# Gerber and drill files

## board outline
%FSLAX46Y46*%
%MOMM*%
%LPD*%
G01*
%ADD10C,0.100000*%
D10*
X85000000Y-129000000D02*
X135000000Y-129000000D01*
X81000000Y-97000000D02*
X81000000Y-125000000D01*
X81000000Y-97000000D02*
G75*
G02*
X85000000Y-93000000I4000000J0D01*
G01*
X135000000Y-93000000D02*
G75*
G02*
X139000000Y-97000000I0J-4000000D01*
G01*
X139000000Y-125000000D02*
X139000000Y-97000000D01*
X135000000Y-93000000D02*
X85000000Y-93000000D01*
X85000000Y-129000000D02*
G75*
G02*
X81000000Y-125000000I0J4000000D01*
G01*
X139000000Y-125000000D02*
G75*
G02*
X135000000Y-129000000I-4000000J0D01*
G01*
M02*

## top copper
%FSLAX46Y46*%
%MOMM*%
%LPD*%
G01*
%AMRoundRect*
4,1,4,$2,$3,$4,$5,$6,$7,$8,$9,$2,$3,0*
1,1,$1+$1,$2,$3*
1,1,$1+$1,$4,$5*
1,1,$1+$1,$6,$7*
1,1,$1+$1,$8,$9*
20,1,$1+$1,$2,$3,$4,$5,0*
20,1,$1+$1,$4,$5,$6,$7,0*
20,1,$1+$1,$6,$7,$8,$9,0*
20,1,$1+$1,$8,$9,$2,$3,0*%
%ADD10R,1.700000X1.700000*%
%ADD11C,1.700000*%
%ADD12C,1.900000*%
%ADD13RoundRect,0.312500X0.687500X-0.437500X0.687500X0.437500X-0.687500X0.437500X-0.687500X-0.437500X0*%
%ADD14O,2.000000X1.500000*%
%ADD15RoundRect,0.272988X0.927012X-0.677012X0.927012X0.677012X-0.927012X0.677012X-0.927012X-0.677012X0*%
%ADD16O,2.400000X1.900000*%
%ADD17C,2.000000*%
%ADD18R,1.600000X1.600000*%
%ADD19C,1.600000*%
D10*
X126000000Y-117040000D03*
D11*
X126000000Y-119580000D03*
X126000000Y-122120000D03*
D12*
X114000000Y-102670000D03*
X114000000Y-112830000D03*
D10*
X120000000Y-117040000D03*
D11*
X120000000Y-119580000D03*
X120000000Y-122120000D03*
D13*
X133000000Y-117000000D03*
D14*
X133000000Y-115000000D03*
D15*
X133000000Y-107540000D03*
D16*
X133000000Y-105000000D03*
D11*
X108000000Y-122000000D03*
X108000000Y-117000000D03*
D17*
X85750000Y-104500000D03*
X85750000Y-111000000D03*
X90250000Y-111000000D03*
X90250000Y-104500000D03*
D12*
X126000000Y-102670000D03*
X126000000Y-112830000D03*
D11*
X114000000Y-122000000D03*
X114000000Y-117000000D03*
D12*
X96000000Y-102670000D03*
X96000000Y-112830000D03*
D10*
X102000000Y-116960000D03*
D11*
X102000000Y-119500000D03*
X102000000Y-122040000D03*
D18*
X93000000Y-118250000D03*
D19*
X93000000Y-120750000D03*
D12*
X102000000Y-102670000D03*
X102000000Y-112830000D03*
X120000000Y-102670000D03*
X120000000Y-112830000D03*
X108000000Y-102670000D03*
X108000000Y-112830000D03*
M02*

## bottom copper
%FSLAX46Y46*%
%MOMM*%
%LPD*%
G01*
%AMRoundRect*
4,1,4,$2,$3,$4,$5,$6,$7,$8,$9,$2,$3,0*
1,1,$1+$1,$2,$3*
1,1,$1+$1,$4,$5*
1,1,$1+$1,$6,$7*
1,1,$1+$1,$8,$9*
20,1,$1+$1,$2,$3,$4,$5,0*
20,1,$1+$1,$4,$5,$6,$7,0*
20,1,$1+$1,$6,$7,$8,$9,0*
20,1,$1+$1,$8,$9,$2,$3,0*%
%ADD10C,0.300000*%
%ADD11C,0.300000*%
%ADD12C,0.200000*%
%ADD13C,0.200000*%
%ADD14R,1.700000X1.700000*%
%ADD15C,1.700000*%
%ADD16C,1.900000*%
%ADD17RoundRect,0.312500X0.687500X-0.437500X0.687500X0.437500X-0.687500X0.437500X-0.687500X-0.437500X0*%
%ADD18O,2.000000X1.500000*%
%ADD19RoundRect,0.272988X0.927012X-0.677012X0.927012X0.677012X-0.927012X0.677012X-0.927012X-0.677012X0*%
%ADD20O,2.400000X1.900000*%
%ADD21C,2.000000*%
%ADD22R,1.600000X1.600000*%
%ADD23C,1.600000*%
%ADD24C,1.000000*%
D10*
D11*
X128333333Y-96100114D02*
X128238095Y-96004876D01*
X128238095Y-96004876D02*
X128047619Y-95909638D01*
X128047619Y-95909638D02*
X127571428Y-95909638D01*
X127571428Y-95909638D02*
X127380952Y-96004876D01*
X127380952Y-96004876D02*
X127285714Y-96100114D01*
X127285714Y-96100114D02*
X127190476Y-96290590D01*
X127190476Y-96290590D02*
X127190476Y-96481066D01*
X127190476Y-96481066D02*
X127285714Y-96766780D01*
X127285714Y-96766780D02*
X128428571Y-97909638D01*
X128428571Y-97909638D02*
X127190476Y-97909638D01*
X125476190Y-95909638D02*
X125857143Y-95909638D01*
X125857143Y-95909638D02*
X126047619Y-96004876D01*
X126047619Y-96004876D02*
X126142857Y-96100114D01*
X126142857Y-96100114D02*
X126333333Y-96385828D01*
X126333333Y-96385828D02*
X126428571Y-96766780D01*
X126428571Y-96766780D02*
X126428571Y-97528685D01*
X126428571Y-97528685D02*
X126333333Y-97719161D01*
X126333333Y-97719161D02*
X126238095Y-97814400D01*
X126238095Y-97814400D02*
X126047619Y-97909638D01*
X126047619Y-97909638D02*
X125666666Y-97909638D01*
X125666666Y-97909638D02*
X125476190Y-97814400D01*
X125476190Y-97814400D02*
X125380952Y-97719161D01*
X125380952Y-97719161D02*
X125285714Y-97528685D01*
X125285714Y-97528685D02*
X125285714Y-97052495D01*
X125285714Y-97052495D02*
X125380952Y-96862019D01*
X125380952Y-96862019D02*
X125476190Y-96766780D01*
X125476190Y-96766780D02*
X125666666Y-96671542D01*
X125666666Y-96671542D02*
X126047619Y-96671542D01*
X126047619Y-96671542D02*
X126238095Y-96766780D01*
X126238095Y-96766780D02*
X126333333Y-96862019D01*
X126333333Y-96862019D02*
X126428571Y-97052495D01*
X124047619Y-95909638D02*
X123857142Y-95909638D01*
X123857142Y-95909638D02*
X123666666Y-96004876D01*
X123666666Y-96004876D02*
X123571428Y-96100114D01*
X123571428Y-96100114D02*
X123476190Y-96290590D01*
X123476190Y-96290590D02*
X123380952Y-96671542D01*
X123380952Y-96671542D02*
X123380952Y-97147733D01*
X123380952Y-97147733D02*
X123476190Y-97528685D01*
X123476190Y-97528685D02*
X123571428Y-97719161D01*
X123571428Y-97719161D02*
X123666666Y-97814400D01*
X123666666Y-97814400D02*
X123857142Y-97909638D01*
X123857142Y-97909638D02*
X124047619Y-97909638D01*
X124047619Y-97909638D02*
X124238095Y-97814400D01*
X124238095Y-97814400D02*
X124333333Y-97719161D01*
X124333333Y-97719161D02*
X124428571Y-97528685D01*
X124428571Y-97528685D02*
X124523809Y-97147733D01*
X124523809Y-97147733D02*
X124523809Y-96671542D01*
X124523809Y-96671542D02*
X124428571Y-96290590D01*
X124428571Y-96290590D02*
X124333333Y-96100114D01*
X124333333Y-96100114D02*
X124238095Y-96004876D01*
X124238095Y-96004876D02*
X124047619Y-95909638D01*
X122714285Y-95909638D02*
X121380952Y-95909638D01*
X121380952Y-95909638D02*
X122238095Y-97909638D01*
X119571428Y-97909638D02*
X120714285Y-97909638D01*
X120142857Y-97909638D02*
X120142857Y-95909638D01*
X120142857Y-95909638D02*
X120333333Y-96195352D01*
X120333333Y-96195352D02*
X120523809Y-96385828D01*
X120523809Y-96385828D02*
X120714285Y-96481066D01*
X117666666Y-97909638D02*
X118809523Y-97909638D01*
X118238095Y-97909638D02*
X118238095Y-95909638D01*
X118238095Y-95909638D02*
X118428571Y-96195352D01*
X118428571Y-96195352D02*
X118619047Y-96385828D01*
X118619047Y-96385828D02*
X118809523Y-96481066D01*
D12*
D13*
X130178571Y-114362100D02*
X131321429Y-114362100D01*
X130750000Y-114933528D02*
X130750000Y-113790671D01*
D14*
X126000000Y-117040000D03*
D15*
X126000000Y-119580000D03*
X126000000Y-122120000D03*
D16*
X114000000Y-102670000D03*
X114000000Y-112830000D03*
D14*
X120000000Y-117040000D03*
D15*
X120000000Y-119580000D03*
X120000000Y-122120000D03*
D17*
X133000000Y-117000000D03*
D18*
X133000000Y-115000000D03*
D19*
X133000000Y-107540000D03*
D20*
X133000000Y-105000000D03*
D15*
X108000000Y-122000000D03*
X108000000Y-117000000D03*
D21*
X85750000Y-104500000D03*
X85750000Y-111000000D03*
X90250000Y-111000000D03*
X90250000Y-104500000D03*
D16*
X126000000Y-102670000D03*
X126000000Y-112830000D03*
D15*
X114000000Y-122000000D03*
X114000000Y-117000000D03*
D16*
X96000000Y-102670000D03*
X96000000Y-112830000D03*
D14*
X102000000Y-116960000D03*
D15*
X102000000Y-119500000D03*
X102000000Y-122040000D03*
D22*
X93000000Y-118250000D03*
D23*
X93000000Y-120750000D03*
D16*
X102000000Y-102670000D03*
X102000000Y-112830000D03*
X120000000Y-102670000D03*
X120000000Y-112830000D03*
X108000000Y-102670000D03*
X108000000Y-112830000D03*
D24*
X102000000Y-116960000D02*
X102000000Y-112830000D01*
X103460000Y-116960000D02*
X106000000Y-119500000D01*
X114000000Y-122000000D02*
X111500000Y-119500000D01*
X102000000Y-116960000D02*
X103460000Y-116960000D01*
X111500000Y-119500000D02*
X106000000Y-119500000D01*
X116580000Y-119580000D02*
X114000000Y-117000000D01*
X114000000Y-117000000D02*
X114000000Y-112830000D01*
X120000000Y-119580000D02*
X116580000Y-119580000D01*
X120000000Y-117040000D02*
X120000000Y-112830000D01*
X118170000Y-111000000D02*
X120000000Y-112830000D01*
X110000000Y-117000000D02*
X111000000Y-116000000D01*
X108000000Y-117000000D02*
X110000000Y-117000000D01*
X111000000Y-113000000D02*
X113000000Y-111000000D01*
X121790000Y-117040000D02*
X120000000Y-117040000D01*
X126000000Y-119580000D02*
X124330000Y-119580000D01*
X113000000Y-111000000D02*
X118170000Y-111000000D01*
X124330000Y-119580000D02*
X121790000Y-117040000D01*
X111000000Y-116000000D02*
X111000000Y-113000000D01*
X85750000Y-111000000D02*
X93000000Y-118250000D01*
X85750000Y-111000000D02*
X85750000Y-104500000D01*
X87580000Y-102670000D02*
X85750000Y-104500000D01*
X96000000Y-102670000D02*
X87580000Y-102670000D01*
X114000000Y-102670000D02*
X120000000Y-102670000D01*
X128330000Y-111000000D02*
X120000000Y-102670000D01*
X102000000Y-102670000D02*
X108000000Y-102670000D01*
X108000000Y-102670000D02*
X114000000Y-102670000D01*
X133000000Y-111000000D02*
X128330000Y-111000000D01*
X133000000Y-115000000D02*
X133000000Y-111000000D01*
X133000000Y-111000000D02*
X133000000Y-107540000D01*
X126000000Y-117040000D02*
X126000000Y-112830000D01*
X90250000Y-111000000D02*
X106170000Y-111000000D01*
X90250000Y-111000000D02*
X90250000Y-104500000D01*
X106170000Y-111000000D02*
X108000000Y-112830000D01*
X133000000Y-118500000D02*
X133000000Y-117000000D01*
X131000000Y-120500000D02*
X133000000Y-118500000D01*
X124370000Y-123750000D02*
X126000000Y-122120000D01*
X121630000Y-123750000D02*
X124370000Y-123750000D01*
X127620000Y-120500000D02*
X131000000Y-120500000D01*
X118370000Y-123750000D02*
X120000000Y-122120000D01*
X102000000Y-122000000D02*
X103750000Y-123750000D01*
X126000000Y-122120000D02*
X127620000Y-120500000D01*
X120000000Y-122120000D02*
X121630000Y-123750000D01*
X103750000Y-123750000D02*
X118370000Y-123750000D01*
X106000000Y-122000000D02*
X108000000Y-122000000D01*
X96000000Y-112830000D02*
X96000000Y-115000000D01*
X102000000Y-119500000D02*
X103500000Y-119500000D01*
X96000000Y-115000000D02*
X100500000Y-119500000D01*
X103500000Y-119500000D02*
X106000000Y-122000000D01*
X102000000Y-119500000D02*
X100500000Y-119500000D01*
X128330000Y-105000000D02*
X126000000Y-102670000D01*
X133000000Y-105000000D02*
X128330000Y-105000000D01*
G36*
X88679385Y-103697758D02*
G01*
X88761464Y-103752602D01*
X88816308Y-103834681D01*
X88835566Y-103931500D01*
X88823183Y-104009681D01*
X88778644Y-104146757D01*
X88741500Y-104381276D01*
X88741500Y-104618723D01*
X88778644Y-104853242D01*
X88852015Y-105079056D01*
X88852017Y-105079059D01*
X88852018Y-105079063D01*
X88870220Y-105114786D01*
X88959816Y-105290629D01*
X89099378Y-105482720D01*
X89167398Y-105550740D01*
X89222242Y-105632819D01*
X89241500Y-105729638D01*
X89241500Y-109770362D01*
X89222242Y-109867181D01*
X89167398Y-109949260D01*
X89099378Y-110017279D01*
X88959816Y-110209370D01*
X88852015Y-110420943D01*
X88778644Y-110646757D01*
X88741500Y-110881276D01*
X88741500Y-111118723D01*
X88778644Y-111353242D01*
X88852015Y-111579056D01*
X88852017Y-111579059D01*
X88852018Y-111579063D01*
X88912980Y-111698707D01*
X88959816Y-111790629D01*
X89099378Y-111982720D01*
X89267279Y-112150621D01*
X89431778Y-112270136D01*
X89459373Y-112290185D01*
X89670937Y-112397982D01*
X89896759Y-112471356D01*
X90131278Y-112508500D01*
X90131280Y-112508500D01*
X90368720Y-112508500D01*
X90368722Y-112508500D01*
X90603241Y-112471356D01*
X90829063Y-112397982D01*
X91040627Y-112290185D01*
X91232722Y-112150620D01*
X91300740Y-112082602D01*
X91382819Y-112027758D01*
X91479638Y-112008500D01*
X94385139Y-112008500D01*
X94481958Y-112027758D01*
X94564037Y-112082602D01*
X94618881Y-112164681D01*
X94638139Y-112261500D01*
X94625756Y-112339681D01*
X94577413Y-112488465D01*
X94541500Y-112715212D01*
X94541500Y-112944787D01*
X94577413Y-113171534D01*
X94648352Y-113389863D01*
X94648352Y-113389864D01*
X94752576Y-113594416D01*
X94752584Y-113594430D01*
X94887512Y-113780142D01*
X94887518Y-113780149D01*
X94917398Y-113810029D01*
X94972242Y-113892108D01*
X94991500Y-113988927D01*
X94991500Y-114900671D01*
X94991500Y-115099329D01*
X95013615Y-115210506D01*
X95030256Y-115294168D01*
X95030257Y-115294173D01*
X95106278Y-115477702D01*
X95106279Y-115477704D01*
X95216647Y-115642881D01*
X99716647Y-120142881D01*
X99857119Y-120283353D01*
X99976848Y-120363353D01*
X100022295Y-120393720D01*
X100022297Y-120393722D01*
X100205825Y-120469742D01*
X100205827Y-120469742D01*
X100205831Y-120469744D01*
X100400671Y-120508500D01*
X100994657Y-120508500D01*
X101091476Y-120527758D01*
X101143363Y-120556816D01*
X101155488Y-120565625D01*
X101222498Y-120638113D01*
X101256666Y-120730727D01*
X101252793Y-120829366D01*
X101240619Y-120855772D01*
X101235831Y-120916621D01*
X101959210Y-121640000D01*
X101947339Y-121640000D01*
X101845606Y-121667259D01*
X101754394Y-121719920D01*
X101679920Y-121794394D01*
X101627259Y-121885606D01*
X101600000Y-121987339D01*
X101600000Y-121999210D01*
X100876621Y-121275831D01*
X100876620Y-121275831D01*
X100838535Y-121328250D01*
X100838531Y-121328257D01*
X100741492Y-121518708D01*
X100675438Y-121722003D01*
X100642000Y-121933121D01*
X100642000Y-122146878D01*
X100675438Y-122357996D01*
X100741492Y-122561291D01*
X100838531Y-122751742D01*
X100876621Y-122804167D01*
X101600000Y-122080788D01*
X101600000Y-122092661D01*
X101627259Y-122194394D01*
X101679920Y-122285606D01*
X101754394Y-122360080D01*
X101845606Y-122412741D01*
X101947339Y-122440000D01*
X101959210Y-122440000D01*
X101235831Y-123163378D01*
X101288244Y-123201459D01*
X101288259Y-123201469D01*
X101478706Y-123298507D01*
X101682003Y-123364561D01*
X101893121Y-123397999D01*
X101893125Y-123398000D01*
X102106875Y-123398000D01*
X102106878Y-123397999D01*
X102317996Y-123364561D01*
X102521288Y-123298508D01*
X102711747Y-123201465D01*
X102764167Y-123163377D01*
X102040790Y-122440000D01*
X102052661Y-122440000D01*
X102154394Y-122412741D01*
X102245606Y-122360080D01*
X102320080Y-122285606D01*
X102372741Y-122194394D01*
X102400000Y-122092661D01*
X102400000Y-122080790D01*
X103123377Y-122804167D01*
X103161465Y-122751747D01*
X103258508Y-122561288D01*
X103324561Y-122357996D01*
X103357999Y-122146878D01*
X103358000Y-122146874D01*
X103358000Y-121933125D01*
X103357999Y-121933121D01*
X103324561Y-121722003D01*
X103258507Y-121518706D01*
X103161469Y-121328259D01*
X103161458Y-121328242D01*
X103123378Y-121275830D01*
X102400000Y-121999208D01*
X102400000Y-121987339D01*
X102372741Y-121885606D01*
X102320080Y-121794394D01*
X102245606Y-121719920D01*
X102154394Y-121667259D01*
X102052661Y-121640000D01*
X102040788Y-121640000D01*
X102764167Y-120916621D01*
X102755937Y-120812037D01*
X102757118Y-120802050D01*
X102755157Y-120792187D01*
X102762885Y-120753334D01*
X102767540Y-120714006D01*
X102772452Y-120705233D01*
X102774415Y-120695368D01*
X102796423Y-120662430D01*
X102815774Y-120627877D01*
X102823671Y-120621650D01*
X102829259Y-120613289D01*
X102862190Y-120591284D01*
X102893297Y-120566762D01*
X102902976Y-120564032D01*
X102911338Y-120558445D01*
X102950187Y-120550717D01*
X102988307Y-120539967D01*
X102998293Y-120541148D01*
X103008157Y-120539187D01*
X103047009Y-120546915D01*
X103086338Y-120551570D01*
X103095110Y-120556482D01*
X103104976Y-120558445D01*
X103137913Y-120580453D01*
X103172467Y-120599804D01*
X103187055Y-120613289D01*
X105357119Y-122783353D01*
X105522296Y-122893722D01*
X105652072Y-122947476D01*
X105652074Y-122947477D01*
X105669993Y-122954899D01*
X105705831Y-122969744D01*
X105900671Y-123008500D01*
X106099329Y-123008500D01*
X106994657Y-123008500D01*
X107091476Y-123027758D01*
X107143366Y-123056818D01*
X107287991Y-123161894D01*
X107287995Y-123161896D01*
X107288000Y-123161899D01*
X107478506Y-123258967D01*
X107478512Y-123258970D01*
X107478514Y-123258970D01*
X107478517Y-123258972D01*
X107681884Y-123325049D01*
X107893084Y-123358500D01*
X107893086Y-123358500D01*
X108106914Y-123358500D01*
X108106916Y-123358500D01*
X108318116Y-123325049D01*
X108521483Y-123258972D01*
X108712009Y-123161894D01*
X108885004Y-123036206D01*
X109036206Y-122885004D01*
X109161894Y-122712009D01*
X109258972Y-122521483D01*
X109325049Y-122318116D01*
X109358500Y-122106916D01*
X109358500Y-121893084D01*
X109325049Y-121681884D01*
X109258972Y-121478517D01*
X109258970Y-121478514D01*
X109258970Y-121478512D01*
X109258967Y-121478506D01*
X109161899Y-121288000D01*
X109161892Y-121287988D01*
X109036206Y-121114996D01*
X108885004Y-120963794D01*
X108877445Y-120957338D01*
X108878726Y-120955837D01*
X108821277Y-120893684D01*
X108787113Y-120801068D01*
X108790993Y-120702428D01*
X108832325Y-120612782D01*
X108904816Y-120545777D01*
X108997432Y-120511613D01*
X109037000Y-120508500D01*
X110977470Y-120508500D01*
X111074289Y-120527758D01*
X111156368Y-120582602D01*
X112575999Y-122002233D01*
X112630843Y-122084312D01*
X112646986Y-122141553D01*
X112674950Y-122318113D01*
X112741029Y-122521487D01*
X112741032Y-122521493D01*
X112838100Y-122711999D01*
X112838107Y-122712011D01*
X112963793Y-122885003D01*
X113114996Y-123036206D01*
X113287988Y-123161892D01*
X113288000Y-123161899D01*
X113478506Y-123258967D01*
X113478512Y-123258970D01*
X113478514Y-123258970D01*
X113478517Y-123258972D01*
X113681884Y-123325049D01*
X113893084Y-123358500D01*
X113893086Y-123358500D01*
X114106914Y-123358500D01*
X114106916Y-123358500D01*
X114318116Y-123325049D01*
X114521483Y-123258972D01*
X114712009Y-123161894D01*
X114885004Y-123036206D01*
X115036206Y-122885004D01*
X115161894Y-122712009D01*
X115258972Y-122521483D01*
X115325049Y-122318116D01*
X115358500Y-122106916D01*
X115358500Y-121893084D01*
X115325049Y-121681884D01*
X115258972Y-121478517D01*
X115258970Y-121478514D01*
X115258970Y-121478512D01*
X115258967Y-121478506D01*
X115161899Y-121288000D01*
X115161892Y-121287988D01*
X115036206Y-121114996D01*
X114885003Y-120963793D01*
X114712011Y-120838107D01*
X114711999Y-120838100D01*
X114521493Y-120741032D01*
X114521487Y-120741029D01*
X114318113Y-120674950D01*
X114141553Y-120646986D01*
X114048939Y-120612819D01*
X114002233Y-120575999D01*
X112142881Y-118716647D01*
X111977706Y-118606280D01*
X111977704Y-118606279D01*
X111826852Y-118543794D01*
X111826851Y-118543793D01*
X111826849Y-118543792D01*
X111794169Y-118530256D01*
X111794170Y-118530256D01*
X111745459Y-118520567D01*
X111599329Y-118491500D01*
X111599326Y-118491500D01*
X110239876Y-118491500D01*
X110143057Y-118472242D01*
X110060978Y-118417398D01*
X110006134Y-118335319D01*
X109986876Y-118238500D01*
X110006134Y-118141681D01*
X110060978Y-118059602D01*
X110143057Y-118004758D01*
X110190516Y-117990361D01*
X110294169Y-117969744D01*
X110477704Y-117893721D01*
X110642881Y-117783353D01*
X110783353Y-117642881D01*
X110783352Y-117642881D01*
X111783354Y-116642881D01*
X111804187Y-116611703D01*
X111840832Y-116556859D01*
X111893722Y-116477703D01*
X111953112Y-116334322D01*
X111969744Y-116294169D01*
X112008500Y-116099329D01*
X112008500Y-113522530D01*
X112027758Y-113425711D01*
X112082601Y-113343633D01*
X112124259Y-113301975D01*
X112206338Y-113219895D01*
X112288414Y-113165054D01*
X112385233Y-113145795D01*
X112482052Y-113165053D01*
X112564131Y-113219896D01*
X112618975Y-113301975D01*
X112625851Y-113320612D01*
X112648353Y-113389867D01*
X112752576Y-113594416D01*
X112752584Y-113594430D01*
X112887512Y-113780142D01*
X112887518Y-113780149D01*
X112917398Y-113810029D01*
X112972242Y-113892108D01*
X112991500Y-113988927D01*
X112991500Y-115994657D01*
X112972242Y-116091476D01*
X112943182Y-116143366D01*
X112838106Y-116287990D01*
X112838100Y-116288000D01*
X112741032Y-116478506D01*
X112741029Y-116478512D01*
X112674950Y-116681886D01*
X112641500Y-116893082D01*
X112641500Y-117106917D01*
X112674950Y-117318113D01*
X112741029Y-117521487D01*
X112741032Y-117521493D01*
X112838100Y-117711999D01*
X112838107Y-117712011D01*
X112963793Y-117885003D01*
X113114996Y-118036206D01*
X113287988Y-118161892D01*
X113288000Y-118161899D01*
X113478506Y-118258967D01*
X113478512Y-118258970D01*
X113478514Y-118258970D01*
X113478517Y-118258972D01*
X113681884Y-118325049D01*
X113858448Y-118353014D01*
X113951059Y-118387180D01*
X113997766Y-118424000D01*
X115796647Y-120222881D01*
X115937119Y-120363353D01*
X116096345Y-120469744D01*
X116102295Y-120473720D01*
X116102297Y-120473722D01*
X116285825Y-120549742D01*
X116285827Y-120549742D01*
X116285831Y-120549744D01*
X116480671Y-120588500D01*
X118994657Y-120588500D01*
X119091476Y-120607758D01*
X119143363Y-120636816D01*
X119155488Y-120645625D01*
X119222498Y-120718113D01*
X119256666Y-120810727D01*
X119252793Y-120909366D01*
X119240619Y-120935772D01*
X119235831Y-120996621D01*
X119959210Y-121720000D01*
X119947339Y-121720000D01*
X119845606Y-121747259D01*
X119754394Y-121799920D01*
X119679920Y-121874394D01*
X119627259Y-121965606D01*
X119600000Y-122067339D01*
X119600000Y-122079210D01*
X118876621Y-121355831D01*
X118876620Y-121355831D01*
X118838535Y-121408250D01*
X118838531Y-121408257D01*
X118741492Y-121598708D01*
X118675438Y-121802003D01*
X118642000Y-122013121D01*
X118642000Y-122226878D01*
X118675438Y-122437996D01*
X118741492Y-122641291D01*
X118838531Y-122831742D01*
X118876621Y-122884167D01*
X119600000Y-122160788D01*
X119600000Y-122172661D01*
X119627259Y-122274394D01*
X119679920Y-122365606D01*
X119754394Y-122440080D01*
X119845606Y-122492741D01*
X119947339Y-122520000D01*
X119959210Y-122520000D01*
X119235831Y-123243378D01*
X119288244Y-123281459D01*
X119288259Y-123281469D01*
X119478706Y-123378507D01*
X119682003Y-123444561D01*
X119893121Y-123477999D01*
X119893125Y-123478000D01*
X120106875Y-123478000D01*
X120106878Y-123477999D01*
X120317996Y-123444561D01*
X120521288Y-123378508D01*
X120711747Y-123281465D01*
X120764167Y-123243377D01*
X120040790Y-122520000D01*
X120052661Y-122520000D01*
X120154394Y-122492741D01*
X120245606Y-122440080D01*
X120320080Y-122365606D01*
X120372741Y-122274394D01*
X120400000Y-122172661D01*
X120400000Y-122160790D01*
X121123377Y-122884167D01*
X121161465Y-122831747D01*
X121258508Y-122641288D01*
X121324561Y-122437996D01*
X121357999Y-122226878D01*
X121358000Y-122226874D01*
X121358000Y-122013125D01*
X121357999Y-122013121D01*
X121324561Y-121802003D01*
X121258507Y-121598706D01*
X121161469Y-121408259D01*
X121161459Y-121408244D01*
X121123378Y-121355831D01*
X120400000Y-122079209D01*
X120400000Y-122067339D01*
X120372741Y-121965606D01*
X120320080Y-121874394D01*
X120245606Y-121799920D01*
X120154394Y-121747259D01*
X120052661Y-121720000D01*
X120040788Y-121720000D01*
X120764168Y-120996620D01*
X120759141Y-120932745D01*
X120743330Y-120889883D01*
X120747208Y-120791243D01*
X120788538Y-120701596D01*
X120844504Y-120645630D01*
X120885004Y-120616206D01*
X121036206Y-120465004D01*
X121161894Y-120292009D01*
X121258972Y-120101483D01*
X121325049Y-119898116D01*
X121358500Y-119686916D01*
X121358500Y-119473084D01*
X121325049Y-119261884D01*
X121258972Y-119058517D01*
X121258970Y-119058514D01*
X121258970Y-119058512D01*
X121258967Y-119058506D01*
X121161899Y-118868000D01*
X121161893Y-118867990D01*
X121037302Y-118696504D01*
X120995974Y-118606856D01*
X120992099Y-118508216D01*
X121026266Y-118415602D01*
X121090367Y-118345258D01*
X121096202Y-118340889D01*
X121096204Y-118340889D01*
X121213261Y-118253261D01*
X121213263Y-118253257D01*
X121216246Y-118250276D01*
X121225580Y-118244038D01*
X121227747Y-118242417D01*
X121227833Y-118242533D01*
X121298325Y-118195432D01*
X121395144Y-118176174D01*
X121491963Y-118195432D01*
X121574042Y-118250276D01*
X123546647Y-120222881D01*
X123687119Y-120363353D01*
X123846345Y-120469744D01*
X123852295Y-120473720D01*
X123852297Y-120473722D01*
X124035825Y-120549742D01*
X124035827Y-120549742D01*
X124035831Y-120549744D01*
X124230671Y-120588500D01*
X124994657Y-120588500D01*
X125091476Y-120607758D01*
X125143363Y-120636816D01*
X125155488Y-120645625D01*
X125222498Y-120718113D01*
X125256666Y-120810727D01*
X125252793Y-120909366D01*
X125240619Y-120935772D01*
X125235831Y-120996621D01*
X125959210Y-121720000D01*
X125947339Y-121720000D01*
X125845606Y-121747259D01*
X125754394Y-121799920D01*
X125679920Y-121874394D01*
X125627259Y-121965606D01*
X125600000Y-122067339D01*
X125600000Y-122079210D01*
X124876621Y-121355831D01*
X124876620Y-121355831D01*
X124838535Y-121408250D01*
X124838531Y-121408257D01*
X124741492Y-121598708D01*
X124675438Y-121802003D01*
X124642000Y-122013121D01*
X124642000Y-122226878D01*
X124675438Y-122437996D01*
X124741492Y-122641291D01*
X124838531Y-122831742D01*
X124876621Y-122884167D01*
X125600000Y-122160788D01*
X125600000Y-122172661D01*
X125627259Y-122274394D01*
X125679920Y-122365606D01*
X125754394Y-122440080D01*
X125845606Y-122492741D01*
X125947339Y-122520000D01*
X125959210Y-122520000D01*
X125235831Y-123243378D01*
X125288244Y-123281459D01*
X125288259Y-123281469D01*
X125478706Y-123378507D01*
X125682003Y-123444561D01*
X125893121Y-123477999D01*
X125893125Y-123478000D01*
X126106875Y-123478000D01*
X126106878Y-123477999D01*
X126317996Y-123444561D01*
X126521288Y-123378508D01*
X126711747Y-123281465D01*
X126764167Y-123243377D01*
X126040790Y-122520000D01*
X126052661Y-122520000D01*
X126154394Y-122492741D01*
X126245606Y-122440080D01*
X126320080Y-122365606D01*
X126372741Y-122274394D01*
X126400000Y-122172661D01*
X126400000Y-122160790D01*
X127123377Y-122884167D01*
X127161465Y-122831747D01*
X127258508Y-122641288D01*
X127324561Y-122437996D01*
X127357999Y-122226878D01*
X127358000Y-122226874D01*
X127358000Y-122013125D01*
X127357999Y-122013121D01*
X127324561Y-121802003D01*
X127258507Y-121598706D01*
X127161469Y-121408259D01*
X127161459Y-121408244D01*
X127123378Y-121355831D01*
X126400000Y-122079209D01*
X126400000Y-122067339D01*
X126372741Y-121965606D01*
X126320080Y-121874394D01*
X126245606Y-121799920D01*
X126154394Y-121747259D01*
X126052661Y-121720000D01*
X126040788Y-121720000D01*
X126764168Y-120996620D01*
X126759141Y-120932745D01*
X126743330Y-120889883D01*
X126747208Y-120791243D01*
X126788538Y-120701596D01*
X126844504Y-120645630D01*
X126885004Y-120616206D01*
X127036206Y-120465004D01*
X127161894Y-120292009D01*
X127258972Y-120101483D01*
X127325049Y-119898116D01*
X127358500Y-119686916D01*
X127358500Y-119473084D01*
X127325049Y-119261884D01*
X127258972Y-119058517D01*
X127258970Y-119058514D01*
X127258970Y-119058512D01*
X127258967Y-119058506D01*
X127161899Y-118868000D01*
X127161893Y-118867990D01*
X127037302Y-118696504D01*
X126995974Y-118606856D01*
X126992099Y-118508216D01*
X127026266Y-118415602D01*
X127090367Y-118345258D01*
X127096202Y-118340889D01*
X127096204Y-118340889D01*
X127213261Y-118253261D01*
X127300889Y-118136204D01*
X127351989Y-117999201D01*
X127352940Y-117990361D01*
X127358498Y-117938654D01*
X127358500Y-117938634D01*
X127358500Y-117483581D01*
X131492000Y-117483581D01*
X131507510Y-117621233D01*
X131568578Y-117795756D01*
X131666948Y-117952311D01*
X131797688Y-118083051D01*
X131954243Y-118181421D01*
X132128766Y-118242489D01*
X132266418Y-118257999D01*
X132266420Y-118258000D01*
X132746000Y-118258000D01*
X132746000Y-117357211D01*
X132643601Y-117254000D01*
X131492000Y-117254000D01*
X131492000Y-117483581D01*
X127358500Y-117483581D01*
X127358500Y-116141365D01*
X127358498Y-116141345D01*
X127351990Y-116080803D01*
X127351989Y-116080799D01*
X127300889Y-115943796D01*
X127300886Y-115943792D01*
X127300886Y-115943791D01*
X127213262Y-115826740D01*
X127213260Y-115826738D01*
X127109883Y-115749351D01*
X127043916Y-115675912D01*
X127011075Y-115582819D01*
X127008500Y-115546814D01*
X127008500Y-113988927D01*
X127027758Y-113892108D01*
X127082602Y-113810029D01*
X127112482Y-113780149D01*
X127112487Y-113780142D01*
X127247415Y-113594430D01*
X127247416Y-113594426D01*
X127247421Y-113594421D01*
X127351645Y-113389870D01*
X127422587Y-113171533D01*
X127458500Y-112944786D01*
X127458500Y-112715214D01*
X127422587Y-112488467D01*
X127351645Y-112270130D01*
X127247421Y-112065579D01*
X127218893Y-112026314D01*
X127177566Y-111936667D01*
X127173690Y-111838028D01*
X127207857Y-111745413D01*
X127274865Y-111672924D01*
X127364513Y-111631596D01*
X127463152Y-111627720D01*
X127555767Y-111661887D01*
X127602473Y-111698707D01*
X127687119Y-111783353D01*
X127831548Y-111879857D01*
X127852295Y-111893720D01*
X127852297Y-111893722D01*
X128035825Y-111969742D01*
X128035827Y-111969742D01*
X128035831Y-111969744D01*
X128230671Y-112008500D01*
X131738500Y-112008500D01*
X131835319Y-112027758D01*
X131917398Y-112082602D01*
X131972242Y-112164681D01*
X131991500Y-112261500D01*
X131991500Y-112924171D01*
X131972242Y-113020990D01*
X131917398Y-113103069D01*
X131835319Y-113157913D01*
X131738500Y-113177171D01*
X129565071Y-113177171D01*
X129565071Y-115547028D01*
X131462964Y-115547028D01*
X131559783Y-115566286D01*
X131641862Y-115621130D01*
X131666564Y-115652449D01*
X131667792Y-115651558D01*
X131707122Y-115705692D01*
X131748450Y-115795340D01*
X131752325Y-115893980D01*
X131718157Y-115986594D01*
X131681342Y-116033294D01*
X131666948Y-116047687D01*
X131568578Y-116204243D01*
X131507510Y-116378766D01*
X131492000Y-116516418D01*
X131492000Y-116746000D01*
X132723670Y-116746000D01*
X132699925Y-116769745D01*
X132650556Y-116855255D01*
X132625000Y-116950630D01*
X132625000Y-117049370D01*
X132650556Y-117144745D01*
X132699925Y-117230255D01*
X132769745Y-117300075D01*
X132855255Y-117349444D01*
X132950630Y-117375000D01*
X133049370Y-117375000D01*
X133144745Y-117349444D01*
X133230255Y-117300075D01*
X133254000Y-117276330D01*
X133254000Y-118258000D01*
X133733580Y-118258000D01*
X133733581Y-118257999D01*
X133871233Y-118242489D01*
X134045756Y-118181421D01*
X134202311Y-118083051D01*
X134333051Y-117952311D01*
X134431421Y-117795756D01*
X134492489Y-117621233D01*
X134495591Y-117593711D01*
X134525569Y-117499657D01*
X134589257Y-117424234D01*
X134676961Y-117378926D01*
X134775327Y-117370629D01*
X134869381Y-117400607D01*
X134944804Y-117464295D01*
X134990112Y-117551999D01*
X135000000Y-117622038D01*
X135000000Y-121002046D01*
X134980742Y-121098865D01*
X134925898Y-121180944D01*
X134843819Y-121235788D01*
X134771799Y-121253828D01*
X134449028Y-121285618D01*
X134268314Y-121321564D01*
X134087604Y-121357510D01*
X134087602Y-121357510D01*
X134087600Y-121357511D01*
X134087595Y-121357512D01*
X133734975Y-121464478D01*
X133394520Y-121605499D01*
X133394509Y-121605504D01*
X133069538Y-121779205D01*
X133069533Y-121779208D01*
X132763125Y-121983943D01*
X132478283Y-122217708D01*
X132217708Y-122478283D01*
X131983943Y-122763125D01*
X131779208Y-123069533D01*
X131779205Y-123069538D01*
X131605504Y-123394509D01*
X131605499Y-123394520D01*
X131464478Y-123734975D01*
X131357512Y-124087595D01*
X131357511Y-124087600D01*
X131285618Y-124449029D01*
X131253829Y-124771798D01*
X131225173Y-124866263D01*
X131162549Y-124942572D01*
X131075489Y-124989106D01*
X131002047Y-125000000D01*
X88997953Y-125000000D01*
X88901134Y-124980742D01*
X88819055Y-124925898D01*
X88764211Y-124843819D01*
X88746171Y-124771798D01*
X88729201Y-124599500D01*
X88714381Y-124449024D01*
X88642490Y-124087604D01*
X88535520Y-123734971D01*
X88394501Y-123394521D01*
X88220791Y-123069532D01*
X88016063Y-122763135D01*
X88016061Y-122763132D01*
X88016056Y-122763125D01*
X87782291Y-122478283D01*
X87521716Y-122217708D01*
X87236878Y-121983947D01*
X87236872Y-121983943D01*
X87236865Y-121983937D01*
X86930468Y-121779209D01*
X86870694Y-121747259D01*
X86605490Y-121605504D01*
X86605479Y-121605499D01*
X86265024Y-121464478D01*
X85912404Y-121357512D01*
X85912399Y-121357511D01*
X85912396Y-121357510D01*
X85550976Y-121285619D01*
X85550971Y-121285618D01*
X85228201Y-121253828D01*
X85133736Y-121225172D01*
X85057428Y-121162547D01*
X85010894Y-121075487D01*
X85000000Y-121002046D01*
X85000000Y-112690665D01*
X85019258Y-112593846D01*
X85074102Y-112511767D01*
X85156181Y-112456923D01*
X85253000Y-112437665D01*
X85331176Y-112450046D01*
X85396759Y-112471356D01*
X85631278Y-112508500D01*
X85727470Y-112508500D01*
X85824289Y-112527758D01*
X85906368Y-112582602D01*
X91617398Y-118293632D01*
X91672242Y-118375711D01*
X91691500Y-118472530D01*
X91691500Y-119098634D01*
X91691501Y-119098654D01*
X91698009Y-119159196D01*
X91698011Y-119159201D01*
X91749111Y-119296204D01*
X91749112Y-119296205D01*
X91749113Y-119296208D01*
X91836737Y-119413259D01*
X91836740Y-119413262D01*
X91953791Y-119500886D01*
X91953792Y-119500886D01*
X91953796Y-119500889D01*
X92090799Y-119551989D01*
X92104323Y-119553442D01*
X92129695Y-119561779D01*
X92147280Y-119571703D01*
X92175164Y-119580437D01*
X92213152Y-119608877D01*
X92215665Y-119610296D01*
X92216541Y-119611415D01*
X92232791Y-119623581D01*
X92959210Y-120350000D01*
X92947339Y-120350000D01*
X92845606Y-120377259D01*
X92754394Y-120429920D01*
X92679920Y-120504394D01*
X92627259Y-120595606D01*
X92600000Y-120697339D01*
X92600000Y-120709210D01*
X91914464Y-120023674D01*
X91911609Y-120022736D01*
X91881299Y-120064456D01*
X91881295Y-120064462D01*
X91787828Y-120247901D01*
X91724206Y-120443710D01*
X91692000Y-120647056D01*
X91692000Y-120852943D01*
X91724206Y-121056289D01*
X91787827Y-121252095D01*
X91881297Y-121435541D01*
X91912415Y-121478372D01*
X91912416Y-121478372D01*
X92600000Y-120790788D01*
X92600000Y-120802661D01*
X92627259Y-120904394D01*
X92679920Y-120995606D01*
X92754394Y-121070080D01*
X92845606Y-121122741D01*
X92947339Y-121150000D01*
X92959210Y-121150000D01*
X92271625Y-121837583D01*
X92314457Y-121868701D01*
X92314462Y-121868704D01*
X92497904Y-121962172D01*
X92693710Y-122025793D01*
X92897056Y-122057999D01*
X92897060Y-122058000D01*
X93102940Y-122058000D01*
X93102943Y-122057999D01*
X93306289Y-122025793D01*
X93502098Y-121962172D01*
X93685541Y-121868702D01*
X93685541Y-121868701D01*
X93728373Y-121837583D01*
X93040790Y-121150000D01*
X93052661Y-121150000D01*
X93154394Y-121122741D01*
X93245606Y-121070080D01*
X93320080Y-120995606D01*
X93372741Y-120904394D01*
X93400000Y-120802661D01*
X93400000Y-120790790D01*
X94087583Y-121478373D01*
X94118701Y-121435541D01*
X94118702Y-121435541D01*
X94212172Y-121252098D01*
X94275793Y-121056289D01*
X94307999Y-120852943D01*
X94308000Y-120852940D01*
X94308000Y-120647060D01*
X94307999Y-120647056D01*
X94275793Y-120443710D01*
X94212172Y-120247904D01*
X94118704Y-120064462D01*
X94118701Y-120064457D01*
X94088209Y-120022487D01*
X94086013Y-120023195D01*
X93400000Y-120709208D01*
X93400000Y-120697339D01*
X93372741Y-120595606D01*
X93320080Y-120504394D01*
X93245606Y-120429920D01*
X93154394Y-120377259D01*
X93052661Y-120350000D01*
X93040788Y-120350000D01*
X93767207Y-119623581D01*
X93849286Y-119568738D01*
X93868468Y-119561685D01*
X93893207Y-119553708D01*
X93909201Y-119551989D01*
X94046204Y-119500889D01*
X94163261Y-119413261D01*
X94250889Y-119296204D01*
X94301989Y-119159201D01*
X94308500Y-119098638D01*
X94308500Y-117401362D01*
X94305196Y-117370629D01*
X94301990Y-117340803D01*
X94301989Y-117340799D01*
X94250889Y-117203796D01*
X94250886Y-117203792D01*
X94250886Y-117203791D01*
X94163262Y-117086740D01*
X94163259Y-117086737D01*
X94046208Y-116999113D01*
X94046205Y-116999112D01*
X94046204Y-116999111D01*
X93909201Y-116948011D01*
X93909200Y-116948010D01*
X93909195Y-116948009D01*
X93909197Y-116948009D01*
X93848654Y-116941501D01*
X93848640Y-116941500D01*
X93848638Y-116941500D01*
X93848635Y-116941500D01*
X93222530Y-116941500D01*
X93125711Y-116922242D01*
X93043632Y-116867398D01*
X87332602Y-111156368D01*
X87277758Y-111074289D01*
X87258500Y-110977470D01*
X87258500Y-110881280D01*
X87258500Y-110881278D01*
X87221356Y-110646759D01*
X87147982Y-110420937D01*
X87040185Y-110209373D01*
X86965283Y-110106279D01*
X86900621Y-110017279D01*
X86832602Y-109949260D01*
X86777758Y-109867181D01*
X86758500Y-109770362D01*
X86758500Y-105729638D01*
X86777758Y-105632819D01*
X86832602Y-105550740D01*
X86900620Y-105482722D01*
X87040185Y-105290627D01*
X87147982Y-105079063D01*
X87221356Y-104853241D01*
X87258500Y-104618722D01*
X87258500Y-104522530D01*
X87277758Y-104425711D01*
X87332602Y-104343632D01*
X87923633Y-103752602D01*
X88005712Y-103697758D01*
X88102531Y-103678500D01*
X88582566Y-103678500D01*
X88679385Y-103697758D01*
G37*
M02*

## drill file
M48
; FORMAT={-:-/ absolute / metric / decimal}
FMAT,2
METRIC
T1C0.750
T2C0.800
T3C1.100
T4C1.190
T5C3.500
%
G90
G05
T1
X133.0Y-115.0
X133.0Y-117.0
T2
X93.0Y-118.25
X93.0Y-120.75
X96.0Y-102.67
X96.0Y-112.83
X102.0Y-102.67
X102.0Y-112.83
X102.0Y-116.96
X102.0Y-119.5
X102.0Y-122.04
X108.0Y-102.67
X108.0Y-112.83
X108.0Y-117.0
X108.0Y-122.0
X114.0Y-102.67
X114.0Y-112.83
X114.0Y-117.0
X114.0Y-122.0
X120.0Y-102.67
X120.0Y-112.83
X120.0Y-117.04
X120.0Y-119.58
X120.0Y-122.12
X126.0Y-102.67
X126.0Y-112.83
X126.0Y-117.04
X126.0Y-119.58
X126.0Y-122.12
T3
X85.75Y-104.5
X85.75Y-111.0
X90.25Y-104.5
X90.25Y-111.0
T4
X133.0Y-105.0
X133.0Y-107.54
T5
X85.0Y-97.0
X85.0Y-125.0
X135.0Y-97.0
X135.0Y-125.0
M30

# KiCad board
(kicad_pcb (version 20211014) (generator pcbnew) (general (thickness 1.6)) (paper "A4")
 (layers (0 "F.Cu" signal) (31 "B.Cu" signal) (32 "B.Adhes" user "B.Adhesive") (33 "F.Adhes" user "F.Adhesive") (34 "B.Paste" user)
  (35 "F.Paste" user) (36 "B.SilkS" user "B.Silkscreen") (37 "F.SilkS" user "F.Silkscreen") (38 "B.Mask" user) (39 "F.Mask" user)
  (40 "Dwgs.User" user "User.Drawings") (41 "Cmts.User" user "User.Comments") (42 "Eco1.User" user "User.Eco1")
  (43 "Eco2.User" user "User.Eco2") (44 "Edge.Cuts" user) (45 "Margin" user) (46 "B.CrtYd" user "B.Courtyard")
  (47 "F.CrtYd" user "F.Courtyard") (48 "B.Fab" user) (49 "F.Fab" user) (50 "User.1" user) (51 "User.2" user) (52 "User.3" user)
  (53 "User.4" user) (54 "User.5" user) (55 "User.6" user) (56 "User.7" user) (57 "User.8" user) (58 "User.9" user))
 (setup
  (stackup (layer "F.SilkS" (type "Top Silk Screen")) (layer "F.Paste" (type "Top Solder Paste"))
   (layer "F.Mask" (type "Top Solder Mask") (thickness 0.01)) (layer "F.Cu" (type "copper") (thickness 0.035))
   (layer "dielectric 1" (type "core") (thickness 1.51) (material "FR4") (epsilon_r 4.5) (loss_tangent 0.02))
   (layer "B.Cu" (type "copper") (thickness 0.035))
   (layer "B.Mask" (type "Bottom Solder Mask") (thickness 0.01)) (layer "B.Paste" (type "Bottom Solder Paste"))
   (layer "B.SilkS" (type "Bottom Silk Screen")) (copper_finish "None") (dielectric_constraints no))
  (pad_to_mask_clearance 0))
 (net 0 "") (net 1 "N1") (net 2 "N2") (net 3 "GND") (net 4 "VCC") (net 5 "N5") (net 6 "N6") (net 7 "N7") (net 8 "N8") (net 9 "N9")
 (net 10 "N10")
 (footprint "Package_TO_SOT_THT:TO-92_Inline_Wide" (layer "F.Cu") (at 126 117.04 -90)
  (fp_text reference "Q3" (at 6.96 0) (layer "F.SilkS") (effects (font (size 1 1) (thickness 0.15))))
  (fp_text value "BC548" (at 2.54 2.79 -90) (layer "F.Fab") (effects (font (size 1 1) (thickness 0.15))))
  (pad "1" thru_hole rect (at 0 0 270) (size 1.7 1.7) (drill 0.8) (layers *.Cu *.Mask) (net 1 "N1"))
  (pad "2" thru_hole circle (at 2.54 0 270) (size 1.7 1.7) (drill 0.8) (layers *.Cu *.Mask) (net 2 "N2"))
  (pad "3" thru_hole circle (at 5.08 0 270) (size 1.7 1.7) (drill 0.8) (layers *.Cu *.Mask) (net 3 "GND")))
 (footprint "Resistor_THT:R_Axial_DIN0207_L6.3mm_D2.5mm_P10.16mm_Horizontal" (layer "F.Cu") (at 114 102.67 -90)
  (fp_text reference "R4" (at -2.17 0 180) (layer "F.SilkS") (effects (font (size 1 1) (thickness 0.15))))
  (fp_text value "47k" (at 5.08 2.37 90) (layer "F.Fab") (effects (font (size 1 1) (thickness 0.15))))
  (pad "1" thru_hole circle (at 0 0 270) (size 1.9 1.9) (drill 0.8) (layers *.Cu *.Mask) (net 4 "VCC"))
  (pad "2" thru_hole circle (at 10.16 0 270) (size 1.9 1.9) (drill 0.8) (layers *.Cu *.Mask) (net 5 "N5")))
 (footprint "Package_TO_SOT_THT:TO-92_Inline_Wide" (layer "F.Cu") (at 120 117.04 -90)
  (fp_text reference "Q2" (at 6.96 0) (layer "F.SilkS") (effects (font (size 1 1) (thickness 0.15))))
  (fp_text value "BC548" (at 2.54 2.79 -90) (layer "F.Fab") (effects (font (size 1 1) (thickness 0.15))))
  (pad "1" thru_hole rect (at 0 0 270) (size 1.7 1.7) (drill 0.8) (layers *.Cu *.Mask) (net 2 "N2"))
  (pad "2" thru_hole circle (at 2.54 0 270) (size 1.7 1.7) (drill 0.8) (layers *.Cu *.Mask) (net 5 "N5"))
  (pad "3" thru_hole circle (at 5.08 0 270) (size 1.7 1.7) (drill 0.8) (layers *.Cu *.Mask) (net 3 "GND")))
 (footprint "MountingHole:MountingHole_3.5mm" (layer "F.Cu") (at 135 125) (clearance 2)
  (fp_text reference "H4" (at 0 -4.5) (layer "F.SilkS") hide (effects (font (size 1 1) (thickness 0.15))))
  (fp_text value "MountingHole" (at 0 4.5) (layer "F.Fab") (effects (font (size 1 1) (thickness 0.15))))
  (pad "" np_thru_hole circle (at 0 0) (size 3.5 3.5) (drill 3.5) (layers *.Cu *.Mask)))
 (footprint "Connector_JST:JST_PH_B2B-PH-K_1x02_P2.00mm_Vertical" (layer "F.Cu") (at 133 117 90)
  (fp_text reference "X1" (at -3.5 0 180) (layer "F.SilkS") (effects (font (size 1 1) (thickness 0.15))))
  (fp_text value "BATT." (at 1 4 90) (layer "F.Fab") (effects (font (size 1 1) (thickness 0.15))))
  (pad "1" thru_hole roundrect (at 0 0 90) (size 1.5 2) (drill 0.75) (layers *.Cu *.Mask) (roundrect_rratio 0.208333) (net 3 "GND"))
  (pad "2" thru_hole oval (at 2 0 90) (size 1.5 2) (drill 0.75) (layers *.Cu *.Mask) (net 4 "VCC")))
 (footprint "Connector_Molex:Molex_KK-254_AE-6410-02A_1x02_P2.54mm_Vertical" (layer "F.Cu") (at 133 107.54 90)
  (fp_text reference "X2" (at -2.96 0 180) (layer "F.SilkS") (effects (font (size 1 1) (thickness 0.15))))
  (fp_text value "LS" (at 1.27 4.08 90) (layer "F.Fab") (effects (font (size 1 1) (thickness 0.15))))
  (pad "1" thru_hole roundrect (at 0 0 90) (size 1.9 2.4) (drill 1.19) (layers *.Cu *.Mask) (roundrect_rratio 0.143678) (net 4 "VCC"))
  (pad "2" thru_hole oval (at 2.54 0 90) (size 1.9 2.4) (drill 1.19) (layers *.Cu *.Mask) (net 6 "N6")))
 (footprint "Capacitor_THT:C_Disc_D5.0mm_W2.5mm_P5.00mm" (layer "F.Cu") (at 108 122 90)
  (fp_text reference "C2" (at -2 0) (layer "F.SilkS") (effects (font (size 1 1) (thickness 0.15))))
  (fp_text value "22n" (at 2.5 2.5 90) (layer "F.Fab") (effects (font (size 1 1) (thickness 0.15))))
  (pad "1" thru_hole circle (at 0 0 90) (size 1.7 1.7) (drill 0.8) (layers *.Cu *.Mask) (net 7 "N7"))
  (pad "2" thru_hole circle (at 5 0 90) (size 1.7 1.7) (drill 0.8) (layers *.Cu *.Mask) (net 2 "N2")))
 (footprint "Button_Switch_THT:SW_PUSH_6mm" (layer "F.Cu") (at 85.75 111 90)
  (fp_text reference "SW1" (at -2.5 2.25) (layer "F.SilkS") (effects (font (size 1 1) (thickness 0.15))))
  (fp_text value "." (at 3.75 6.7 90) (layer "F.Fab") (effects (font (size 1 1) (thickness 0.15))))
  (pad "1" thru_hole circle (at 6.5 0 180) (size 2 2) (drill 1.1) (layers *.Cu *.Mask) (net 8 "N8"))
  (pad "1" thru_hole circle (at 0 0 180) (size 2 2) (drill 1.1) (layers *.Cu *.Mask) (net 8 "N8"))
  (pad "2" thru_hole circle (at 0 4.5 180) (size 2 2) (drill 1.1) (layers *.Cu *.Mask) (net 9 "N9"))
  (pad "2" thru_hole circle (at 6.5 4.5 180) (size 2 2) (drill 1.1) (layers *.Cu *.Mask) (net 9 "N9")))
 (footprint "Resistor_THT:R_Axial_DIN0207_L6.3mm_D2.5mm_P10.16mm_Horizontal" (layer "F.Cu") (at 126 102.67 -90)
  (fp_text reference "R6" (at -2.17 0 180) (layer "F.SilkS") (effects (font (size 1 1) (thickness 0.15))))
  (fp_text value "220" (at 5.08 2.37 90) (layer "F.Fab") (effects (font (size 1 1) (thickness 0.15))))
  (pad "1" thru_hole circle (at 0 0 270) (size 1.9 1.9) (drill 0.8) (layers *.Cu *.Mask) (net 6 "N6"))
  (pad "2" thru_hole circle (at 10.16 0 270) (size 1.9 1.9) (drill 0.8) (layers *.Cu *.Mask) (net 1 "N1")))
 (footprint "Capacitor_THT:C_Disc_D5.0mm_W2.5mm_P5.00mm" (layer "F.Cu") (at 114 122 90)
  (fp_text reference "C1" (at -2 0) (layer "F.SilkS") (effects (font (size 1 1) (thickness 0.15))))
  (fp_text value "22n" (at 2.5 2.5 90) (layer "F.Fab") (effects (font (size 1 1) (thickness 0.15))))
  (pad "1" thru_hole circle (at 0 0 90) (size 1.7 1.7) (drill 0.8) (layers *.Cu *.Mask) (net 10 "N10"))
  (pad "2" thru_hole circle (at 5 0 90) (size 1.7 1.7) (drill 0.8) (layers *.Cu *.Mask) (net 5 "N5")))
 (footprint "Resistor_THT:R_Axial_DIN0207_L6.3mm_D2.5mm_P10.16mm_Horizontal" (layer "F.Cu") (at 96 102.67 -90)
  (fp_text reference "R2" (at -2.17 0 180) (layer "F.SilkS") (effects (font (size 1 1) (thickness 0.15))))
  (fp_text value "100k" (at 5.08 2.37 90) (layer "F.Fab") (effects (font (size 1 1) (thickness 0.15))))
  (pad "1" thru_hole circle (at 0 0 270) (size 1.9 1.9) (drill 0.8) (layers *.Cu *.Mask) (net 8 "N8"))
  (pad "2" thru_hole circle (at 10.16 0 270) (size 1.9 1.9) (drill 0.8) (layers *.Cu *.Mask) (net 7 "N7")))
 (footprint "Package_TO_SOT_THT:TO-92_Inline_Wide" (layer "F.Cu") (at 102 116.96 -90)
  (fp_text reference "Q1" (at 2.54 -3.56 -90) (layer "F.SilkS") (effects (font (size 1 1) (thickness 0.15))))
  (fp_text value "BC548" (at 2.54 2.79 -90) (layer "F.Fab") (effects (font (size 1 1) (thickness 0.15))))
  (pad "1" thru_hole rect (at 0 0 270) (size 1.7 1.7) (drill 0.8) (layers *.Cu *.Mask) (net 10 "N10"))
  (pad "2" thru_hole circle (at 2.54 0 270) (size 1.7 1.7) (drill 0.8) (layers *.Cu *.Mask) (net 7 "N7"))
  (pad "3" thru_hole circle (at 5.08 0 270) (size 1.7 1.7) (drill 0.8) (layers *.Cu *.Mask) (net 3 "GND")))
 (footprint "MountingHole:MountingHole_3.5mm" (layer "F.Cu") (at 85 97) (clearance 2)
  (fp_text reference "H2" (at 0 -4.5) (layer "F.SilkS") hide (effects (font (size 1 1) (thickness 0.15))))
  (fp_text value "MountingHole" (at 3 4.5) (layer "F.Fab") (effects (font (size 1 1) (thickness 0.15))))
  (pad "" np_thru_hole circle (at 0 0) (size 3.5 3.5) (drill 3.5) (layers *.Cu *.Mask)))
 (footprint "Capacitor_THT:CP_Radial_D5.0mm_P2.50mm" (layer "F.Cu") (at 93 118.25 -90)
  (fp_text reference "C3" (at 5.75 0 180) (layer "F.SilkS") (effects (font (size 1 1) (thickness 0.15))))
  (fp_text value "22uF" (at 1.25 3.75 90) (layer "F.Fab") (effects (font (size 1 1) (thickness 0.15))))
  (pad "1" thru_hole rect (at 0 0 270) (size 1.6 1.6) (drill 0.8) (layers *.Cu *.Mask) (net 8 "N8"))
  (pad "2" thru_hole circle (at 2.5 0 270) (size 1.6 1.6) (drill 0.8) (layers *.Cu *.Mask) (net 3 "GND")))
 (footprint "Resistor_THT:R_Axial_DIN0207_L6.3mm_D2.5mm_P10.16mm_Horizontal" (layer "F.Cu") (at 102 102.67 -90)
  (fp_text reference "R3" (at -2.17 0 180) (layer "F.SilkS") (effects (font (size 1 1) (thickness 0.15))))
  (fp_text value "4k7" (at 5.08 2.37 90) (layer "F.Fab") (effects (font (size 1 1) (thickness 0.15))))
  (pad "1" thru_hole circle (at 0 0 270) (size 1.9 1.9) (drill 0.8) (layers *.Cu *.Mask) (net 4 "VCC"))
  (pad "2" thru_hole circle (at 10.16 0 270) (size 1.9 1.9) (drill 0.8) (layers *.Cu *.Mask) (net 10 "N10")))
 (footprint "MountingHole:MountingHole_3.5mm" (layer "F.Cu") (at 85 125) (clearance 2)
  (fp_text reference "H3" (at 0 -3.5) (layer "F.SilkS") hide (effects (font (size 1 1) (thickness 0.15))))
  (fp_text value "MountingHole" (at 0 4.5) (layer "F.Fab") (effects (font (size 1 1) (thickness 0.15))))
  (pad "" np_thru_hole circle (at 0 0) (size 3.5 3.5) (drill 3.5) (layers *.Cu *.Mask)))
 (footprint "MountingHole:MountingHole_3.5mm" (layer "F.Cu") (at 135 97) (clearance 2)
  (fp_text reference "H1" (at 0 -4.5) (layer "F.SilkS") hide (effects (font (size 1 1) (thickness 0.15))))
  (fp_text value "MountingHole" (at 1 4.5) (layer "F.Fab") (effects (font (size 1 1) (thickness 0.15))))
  (pad "" np_thru_hole circle (at 0 0) (size 3.5 3.5) (drill 3.5) (layers *.Cu *.Mask)))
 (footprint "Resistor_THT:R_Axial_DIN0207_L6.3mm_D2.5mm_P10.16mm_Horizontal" (layer "F.Cu") (at 120 102.67 -90)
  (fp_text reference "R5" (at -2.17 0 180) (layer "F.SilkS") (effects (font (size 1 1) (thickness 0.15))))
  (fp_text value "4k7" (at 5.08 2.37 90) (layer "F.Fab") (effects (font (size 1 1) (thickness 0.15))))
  (pad "1" thru_hole circle (at 0 0 270) (size 1.9 1.9) (drill 0.8) (layers *.Cu *.Mask) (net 4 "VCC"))
  (pad "2" thru_hole circle (at 10.16 0 270) (size 1.9 1.9) (drill 0.8) (layers *.Cu *.Mask) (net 2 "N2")))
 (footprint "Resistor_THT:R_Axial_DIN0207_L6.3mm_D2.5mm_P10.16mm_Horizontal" (layer "F.Cu") (at 108 102.67 -90)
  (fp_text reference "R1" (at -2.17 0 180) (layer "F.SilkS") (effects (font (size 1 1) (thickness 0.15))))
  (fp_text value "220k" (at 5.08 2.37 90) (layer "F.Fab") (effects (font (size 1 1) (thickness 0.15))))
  (pad "1" thru_hole circle (at 0 0 270) (size 1.9 1.9) (drill 0.8) (layers *.Cu *.Mask) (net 4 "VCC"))
  (pad "2" thru_hole circle (at 10.16 0 270) (size 1.9 1.9) (drill 0.8) (layers *.Cu *.Mask) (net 9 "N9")))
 (gr_line (start 85 129) (end 135 129) (layer "Edge.Cuts") (width 0.1))
 (gr_line (start 81 97) (end 81 125) (layer "Edge.Cuts") (width 0.1))
 (gr_arc (start 81 97) (mid 82.171573 94.171573) (end 85 93) (layer "Edge.Cuts") (width 0.1))
 (gr_arc (start 135 93) (mid 137.828427 94.171573) (end 139 97) (layer "Edge.Cuts") (width 0.1))
 (gr_line (start 139 125) (end 139 97) (layer "Edge.Cuts") (width 0.1))
 (gr_line (start 135 93) (end 85 93) (layer "Edge.Cuts") (width 0.1))
 (gr_arc (start 85 129) (mid 82.171573 127.828427) (end 81 125) (layer "Edge.Cuts") (width 0.1))
 (gr_arc (start 139 125) (mid 137.828427 127.828427) (end 135 129) (layer "Edge.Cuts") (width 0.1))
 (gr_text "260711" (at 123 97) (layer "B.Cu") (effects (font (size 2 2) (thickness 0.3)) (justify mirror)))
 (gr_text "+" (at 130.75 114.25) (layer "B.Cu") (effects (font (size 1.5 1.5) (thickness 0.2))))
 (segment (start 102 116.96) (end 102 112.83) (width 1) (layer "B.Cu") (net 10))
 (segment (start 103.46 116.96) (end 106 119.5) (width 1) (layer "B.Cu") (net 10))
 (segment (start 114 122) (end 111.5 119.5) (width 1) (layer "B.Cu") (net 10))
 (segment (start 102 116.96) (end 103.46 116.96) (width 1) (layer "B.Cu") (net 10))
 (segment (start 111.5 119.5) (end 106 119.5) (width 1) (layer "B.Cu") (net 10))
 (segment (start 116.58 119.58) (end 114 117) (width 1) (layer "B.Cu") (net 5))
 (segment (start 114 117) (end 114 112.83) (width 1) (layer "B.Cu") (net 5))
 (segment (start 120 119.58) (end 116.58 119.58) (width 1) (layer "B.Cu") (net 5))
 (segment (start 120 117.04) (end 120 112.83) (width 1) (layer "B.Cu") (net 2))
 (segment (start 118.17 111) (end 120 112.83) (width 1) (layer "B.Cu") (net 2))
 (segment (start 110 117) (end 111 116) (width 1) (layer "B.Cu") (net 2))
 (segment (start 108 117) (end 110 117) (width 1) (layer "B.Cu") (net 2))
 (segment (start 111 113) (end 113 111) (width 1) (layer "B.Cu") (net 2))
 (segment (start 121.79 117.04) (end 120 117.04) (width 1) (layer "B.Cu") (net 2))
 (segment (start 126 119.58) (end 124.33 119.58) (width 1) (layer "B.Cu") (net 2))
 (segment (start 113 111) (end 118.17 111) (width 1) (layer "B.Cu") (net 2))
 (segment (start 124.33 119.58) (end 121.79 117.04) (width 1) (layer "B.Cu") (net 2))
 (segment (start 111 116) (end 111 113) (width 1) (layer "B.Cu") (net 2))
 (segment (start 85.75 111) (end 93 118.25) (width 1) (layer "B.Cu") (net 8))
 (segment (start 85.75 111) (end 85.75 104.5) (width 1) (layer "B.Cu") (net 8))
 (segment (start 87.58 102.67) (end 85.75 104.5) (width 1) (layer "B.Cu") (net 8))
 (segment (start 96 102.67) (end 87.58 102.67) (width 1) (layer "B.Cu") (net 8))
 (segment (start 114 102.67) (end 120 102.67) (width 1) (layer "B.Cu") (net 4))
 (segment (start 128.33 111) (end 120 102.67) (width 1) (layer "B.Cu") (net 4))
 (segment (start 102 102.67) (end 108 102.67) (width 1) (layer "B.Cu") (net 4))
 (segment (start 108 102.67) (end 114 102.67) (width 1) (layer "B.Cu") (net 4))
 (segment (start 133 111) (end 128.33 111) (width 1) (layer "B.Cu") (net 4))
 (segment (start 133 115) (end 133 111) (width 1) (layer "B.Cu") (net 4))
 (segment (start 133 111) (end 133 107.54) (width 1) (layer "B.Cu") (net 4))
 (segment (start 126 117.04) (end 126 112.83) (width 1) (layer "B.Cu") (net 1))
 (segment (start 90.25 111) (end 106.17 111) (width 1) (layer "B.Cu") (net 9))
 (segment (start 90.25 111) (end 90.25 104.5) (width 1) (layer "B.Cu") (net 9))
 (segment (start 106.17 111) (end 108 112.83) (width 1) (layer "B.Cu") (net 9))
 (segment (start 133 118.5) (end 133 117) (width 1) (layer "B.Cu") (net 3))
 (segment (start 131 120.5) (end 133 118.5) (width 1) (layer "B.Cu") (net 3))
 (segment (start 124.37 123.75) (end 126 122.12) (width 1) (layer "B.Cu") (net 3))
 (segment (start 121.63 123.75) (end 124.37 123.75) (width 1) (layer "B.Cu") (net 3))
 (segment (start 127.62 120.5) (end 131 120.5) (width 1) (layer "B.Cu") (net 3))
 (segment (start 118.37 123.75) (end 120 122.12) (width 1) (layer "B.Cu") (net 3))
 (segment (start 102 122) (end 103.75 123.75) (width 1) (layer "B.Cu") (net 3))
 (segment (start 126 122.12) (end 127.62 120.5) (width 1) (layer "B.Cu") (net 3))
 (segment (start 120 122.12) (end 121.63 123.75) (width 1) (layer "B.Cu") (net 3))
 (segment (start 103.75 123.75) (end 118.37 123.75) (width 1) (layer "B.Cu") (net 3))
 (segment (start 106 122) (end 108 122) (width 1) (layer "B.Cu") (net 7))
 (segment (start 96 112.83) (end 96 115) (width 1) (layer "B.Cu") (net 7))
 (segment (start 102 119.5) (end 103.5 119.5) (width 1) (layer "B.Cu") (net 7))
 (segment (start 96 115) (end 100.5 119.5) (width 1) (layer "B.Cu") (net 7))
 (segment (start 103.5 119.5) (end 106 122) (width 1) (layer "B.Cu") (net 7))
 (segment (start 102 119.5) (end 100.5 119.5) (width 1) (layer "B.Cu") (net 7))
 (segment (start 128.33 105) (end 126 102.67) (width 1) (layer "B.Cu") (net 6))
 (segment (start 133 105) (end 128.33 105) (width 1) (layer "B.Cu") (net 6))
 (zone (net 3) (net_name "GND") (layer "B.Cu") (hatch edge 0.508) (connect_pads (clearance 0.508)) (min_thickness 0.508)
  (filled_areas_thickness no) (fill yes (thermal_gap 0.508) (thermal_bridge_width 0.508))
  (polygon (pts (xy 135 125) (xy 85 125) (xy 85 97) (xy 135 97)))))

